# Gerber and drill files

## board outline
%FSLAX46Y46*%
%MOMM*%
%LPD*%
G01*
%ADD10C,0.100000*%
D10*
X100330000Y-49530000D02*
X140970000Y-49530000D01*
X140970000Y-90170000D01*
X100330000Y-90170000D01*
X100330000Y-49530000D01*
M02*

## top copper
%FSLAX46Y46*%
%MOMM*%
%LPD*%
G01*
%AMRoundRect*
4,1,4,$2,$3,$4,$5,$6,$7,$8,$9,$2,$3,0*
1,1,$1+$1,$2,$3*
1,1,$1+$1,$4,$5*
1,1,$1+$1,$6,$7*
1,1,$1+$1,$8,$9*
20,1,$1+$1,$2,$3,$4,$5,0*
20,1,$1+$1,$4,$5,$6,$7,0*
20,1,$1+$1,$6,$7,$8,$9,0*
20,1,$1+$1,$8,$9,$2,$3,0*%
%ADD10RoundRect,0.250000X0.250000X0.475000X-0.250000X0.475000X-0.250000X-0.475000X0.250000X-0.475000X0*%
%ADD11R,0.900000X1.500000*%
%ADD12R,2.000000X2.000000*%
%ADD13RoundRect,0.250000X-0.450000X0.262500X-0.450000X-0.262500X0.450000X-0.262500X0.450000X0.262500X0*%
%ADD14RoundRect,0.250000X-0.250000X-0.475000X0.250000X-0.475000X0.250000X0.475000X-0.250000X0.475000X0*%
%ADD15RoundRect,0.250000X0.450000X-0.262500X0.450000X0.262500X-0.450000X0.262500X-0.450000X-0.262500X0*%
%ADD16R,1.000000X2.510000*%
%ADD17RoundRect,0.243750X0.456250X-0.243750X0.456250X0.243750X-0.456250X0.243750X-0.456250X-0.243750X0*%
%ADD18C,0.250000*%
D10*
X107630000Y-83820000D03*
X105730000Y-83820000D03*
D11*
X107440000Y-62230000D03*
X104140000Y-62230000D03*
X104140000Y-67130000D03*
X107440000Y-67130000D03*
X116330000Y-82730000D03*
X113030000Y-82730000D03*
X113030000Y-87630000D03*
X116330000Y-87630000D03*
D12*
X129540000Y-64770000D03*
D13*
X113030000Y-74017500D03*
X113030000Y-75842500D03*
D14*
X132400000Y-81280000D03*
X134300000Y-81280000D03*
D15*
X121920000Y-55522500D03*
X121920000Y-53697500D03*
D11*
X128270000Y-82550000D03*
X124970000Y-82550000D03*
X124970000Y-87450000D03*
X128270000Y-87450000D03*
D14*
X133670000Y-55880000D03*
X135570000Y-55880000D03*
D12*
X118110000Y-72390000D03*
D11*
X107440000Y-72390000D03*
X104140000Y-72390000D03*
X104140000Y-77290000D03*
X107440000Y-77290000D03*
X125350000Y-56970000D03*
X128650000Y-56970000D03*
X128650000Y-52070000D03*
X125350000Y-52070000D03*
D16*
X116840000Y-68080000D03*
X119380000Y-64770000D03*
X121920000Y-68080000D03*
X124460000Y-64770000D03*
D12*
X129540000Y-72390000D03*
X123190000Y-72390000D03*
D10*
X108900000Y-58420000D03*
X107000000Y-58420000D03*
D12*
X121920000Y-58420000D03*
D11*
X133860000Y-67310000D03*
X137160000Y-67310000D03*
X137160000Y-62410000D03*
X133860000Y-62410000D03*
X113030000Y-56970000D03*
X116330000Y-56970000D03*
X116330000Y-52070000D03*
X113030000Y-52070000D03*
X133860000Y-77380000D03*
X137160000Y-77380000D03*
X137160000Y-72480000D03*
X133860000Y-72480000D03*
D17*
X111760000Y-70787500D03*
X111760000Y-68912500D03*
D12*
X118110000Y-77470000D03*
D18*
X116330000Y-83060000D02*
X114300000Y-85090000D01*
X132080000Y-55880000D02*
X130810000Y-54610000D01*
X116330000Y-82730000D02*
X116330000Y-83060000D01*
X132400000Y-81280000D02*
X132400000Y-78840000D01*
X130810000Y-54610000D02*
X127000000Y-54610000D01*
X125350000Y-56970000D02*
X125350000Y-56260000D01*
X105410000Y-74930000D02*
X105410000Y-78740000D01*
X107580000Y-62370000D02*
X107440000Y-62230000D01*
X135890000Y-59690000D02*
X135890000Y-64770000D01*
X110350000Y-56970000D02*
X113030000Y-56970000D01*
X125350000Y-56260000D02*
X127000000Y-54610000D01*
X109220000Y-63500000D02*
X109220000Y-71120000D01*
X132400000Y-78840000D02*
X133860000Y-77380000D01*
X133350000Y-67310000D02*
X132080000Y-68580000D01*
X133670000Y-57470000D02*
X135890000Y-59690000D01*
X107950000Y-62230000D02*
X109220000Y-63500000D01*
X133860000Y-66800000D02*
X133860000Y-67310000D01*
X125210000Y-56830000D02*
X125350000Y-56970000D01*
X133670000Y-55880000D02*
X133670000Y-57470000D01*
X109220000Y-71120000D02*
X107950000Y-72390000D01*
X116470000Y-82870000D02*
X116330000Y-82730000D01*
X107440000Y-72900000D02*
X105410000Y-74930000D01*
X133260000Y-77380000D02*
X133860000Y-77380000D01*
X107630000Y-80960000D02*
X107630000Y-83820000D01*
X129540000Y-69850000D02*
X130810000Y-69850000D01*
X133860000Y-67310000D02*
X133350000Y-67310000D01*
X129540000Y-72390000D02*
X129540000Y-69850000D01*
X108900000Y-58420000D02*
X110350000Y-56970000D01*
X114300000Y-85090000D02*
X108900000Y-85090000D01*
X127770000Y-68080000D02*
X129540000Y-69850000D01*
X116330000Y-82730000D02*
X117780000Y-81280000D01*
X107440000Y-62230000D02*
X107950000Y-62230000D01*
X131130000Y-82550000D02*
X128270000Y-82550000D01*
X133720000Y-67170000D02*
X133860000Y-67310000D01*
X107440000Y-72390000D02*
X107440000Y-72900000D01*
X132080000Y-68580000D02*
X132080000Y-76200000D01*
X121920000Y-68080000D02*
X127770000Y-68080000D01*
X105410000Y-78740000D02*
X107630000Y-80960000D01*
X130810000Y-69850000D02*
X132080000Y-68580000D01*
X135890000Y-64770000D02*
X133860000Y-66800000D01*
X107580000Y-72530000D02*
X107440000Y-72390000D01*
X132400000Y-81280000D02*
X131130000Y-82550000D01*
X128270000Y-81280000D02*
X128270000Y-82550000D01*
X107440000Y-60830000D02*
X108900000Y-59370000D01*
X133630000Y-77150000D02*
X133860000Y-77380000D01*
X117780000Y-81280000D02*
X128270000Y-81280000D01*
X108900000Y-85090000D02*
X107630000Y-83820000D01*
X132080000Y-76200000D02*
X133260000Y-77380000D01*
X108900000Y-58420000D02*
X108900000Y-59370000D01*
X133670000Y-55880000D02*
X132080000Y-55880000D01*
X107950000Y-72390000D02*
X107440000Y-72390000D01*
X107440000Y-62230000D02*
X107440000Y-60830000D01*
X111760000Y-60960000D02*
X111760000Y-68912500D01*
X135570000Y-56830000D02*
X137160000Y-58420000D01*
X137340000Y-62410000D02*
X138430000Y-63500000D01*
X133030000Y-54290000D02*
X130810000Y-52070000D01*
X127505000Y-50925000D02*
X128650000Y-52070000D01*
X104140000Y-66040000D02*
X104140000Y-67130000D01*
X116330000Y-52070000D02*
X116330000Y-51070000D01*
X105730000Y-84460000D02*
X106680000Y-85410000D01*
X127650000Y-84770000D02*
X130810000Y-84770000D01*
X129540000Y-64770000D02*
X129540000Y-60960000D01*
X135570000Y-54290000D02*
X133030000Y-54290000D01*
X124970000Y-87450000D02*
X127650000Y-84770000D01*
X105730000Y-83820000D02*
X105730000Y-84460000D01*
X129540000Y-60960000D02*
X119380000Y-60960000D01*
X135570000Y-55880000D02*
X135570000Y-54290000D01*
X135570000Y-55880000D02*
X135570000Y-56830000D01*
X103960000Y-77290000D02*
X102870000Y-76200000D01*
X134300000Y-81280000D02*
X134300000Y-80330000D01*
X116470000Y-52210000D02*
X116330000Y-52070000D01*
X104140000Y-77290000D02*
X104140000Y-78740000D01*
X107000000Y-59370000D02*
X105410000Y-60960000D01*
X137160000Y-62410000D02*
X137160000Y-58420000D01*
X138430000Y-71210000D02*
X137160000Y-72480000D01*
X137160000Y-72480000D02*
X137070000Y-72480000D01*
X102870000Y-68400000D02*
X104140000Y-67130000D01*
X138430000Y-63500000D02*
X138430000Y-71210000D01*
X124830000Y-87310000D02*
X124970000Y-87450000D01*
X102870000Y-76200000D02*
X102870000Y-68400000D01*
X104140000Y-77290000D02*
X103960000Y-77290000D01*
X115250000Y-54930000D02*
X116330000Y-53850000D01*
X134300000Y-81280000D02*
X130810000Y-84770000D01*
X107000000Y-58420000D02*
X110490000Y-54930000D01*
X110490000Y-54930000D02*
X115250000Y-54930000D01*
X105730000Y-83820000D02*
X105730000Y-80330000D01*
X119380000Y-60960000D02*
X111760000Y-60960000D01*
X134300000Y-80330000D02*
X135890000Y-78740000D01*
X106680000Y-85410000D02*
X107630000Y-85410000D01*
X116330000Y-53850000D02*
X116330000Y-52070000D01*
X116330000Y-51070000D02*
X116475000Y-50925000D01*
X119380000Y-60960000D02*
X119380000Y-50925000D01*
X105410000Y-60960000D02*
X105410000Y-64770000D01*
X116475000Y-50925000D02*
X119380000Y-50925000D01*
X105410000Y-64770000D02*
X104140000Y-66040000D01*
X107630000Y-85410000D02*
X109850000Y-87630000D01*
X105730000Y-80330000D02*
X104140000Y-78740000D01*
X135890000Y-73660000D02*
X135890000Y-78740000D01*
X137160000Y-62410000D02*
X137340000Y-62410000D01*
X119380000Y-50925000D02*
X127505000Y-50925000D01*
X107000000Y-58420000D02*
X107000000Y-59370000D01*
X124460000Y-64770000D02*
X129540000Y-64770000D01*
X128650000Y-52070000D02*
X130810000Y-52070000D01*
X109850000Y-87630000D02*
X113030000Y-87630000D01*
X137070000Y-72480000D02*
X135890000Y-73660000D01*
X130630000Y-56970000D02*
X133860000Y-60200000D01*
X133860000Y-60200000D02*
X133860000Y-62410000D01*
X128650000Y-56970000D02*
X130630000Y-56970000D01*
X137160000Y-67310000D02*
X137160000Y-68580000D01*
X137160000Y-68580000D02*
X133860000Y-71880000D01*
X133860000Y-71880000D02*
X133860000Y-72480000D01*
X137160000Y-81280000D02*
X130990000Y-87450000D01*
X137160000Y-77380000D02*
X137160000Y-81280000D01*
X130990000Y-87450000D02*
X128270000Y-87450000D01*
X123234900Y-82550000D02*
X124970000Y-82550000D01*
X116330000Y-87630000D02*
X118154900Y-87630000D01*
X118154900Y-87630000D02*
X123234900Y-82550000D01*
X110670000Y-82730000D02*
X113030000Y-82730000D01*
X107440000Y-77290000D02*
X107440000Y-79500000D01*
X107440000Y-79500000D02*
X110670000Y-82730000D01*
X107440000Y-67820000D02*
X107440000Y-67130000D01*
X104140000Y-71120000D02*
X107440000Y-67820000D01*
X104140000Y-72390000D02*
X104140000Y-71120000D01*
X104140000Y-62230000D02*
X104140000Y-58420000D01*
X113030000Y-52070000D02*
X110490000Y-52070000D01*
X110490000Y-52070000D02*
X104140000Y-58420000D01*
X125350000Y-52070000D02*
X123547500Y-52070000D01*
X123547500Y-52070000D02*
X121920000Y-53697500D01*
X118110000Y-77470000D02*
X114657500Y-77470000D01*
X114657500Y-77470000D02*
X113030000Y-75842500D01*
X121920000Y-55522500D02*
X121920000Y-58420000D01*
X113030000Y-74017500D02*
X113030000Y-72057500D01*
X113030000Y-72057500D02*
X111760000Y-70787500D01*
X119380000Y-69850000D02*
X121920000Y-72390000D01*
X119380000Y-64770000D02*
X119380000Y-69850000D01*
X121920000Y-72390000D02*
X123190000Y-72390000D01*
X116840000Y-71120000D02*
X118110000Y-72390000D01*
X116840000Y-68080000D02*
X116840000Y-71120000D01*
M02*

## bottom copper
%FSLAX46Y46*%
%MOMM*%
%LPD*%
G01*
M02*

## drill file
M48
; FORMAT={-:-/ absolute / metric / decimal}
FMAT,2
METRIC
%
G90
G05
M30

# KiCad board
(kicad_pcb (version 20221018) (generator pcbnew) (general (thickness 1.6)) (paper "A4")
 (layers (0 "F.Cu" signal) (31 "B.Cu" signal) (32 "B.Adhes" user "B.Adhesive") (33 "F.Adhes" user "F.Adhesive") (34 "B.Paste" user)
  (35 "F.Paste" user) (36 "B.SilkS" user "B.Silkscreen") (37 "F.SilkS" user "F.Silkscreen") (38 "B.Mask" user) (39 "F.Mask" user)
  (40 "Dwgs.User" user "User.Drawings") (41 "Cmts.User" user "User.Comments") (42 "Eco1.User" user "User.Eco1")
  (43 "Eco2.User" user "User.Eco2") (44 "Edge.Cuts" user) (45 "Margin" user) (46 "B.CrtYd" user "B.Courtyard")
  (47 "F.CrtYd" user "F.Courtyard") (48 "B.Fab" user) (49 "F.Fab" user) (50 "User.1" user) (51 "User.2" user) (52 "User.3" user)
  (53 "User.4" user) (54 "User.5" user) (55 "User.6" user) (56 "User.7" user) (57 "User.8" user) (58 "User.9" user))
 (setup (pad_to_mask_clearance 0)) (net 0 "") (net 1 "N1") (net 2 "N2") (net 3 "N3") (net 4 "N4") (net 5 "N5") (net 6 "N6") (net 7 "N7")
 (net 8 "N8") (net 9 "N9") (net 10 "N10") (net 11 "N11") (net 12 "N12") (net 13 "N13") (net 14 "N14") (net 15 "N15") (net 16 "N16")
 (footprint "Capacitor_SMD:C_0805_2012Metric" (layer "F.Cu") (at 106.68 83.82 180)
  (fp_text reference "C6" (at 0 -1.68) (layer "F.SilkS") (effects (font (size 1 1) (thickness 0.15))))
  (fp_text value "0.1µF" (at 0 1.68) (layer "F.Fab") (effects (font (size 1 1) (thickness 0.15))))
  (pad "1" smd roundrect (at -0.95 0 180) (size 1 1.45) (layers "F.Cu" "F.Paste" "F.Mask") (roundrect_rratio 0.25) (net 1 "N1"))
  (pad "2" smd roundrect (at 0.95 0 180) (size 1 1.45) (layers "F.Cu" "F.Paste" "F.Mask") (roundrect_rratio 0.25) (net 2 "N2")))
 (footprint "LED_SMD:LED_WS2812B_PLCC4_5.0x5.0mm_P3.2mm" (layer "F.Cu") (at 105.79 64.68 -90)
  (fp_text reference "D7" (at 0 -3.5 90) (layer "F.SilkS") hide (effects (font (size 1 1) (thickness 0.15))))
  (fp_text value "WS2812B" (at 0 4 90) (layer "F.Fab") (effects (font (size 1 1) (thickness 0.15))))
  (pad "1" smd rect (at -2.45 -1.65 270) (size 1.5 0.9) (layers "F.Cu" "F.Paste" "F.Mask") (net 1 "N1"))
  (pad "2" smd rect (at -2.45 1.65 270) (size 1.5 0.9) (layers "F.Cu" "F.Paste" "F.Mask") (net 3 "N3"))
  (pad "3" smd rect (at 2.45 1.65 270) (size 1.5 0.9) (layers "F.Cu" "F.Paste" "F.Mask") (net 2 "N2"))
  (pad "4" smd rect (at 2.45 -1.65 270) (size 1.5 0.9) (layers "F.Cu" "F.Paste" "F.Mask") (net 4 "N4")))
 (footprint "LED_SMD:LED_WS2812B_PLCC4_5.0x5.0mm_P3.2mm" (layer "F.Cu") (at 114.68 85.18 -90)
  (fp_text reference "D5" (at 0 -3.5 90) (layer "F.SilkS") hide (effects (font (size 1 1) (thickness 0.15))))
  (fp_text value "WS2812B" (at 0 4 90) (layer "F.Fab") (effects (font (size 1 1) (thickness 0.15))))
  (pad "1" smd rect (at -2.45 -1.65 270) (size 1.5 0.9) (layers "F.Cu" "F.Paste" "F.Mask") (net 1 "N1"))
  (pad "2" smd rect (at -2.45 1.65 270) (size 1.5 0.9) (layers "F.Cu" "F.Paste" "F.Mask") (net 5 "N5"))
  (pad "3" smd rect (at 2.45 1.65 270) (size 1.5 0.9) (layers "F.Cu" "F.Paste" "F.Mask") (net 2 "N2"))
  (pad "4" smd rect (at 2.45 -1.65 270) (size 1.5 0.9) (layers "F.Cu" "F.Paste" "F.Mask") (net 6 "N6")))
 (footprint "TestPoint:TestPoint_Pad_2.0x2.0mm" (layer "F.Cu") (at 129.54 64.77)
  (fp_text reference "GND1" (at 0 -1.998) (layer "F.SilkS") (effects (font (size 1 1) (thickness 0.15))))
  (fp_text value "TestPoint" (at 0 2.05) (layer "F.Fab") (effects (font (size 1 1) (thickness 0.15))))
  (pad "1" smd rect (at 0 0) (size 2 2) (layers "F.Cu" "F.Mask") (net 2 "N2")))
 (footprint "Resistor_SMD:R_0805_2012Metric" (layer "F.Cu") (at 113.03 74.93 -90)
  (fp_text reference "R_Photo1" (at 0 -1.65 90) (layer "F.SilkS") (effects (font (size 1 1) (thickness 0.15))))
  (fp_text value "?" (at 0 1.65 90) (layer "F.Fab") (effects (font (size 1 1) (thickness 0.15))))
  (pad "1" smd roundrect (at -0.9125 0 270) (size 1.025 1.4) (layers "F.Cu" "F.Paste" "F.Mask") (roundrect_rratio 0.243902) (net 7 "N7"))
  (pad "2" smd roundrect (at 0.9125 0 270) (size 1.025 1.4) (layers "F.Cu" "F.Paste" "F.Mask") (roundrect_rratio 0.243902) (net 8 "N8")))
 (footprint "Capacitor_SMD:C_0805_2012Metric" (layer "F.Cu") (at 133.35 81.28)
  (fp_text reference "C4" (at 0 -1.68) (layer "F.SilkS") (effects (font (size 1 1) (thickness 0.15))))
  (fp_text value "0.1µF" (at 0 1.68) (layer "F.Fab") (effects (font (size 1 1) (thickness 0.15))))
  (pad "1" smd roundrect (at -0.95 0) (size 1 1.45) (layers "F.Cu" "F.Paste" "F.Mask") (roundrect_rratio 0.25) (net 1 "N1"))
  (pad "2" smd roundrect (at 0.95 0) (size 1 1.45) (layers "F.Cu" "F.Paste" "F.Mask") (roundrect_rratio 0.25) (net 2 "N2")))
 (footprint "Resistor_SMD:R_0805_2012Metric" (layer "F.Cu") (at 121.92 54.61 90)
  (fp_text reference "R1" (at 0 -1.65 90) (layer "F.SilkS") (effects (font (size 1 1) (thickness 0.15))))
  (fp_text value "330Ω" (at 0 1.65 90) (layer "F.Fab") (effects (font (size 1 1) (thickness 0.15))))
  (pad "1" smd roundrect (at -0.9125 0 90) (size 1.025 1.4) (layers "F.Cu" "F.Paste" "F.Mask") (roundrect_rratio 0.243902) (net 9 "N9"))
  (pad "2" smd roundrect (at 0.9125 0 90) (size 1.025 1.4) (layers "F.Cu" "F.Paste" "F.Mask") (roundrect_rratio 0.243902) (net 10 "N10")))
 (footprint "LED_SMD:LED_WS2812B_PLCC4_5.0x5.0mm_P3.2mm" (layer "F.Cu") (at 126.62 85 -90)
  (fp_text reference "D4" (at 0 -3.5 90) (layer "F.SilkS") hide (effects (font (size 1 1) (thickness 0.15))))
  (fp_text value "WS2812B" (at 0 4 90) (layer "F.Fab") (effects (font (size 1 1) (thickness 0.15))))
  (pad "1" smd rect (at -2.45 -1.65 270) (size 1.5 0.9) (layers "F.Cu" "F.Paste" "F.Mask") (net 1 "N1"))
  (pad "2" smd rect (at -2.45 1.65 270) (size 1.5 0.9) (layers "F.Cu" "F.Paste" "F.Mask") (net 6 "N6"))
  (pad "3" smd rect (at 2.45 1.65 270) (size 1.5 0.9) (layers "F.Cu" "F.Paste" "F.Mask") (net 2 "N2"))
  (pad "4" smd rect (at 2.45 -1.65 270) (size 1.5 0.9) (layers "F.Cu" "F.Paste" "F.Mask") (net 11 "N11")))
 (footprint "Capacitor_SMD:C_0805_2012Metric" (layer "F.Cu") (at 134.62 55.88)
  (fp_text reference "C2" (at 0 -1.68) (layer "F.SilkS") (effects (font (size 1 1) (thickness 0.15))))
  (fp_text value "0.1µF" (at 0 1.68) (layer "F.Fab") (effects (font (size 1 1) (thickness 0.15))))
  (pad "1" smd roundrect (at -0.95 0) (size 1 1.45) (layers "F.Cu" "F.Paste" "F.Mask") (roundrect_rratio 0.25) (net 1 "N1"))
  (pad "2" smd roundrect (at 0.95 0) (size 1 1.45) (layers "F.Cu" "F.Paste" "F.Mask") (roundrect_rratio 0.25) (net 2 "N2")))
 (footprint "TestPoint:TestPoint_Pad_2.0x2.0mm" (layer "F.Cu") (at 118.11 72.39)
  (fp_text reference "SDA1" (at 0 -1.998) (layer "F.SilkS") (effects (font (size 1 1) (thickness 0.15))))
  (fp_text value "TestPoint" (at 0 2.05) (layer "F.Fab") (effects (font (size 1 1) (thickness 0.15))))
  (pad "1" smd rect (at 0 0) (size 2 2) (layers "F.Cu" "F.Mask") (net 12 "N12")))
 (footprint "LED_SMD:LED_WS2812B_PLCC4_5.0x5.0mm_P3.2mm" (layer "F.Cu") (at 105.79 74.84 -90)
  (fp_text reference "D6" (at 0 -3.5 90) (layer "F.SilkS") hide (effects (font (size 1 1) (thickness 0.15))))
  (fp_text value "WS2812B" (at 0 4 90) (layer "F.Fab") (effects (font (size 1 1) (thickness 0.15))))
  (pad "1" smd rect (at -2.45 -1.65 270) (size 1.5 0.9) (layers "F.Cu" "F.Paste" "F.Mask") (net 1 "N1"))
  (pad "2" smd rect (at -2.45 1.65 270) (size 1.5 0.9) (layers "F.Cu" "F.Paste" "F.Mask") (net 4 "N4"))
  (pad "3" smd rect (at 2.45 1.65 270) (size 1.5 0.9) (layers "F.Cu" "F.Paste" "F.Mask") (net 2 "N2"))
  (pad "4" smd rect (at 2.45 -1.65 270) (size 1.5 0.9) (layers "F.Cu" "F.Paste" "F.Mask") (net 5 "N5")))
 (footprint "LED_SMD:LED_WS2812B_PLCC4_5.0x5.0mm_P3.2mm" (layer "F.Cu") (at 127 54.52 90)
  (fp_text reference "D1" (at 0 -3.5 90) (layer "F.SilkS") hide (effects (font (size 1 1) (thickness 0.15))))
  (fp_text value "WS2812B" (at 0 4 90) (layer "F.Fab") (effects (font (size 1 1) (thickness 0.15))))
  (pad "1" smd rect (at -2.45 -1.65 90) (size 1.5 0.9) (layers "F.Cu" "F.Paste" "F.Mask") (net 1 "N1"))
  (pad "2" smd rect (at -2.45 1.65 90) (size 1.5 0.9) (layers "F.Cu" "F.Paste" "F.Mask") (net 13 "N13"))
  (pad "3" smd rect (at 2.45 1.65 90) (size 1.5 0.9) (layers "F.Cu" "F.Paste" "F.Mask") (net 2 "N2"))
  (pad "4" smd rect (at 2.45 -1.65 90) (size 1.5 0.9) (layers "F.Cu" "F.Paste" "F.Mask") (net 10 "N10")))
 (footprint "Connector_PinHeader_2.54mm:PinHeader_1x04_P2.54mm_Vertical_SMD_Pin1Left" (layer "F.Cu") (at 120.65 66.425 90)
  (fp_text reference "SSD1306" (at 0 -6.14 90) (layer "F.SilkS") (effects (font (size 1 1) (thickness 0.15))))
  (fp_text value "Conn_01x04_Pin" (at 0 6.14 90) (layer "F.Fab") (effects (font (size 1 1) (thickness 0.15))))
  (pad "1" smd rect (at -1.655 -3.81 90) (size 2.51 1) (layers "F.Cu" "F.Paste" "F.Mask") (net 12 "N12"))
  (pad "2" smd rect (at 1.655 -1.27 90) (size 2.51 1) (layers "F.Cu" "F.Paste" "F.Mask") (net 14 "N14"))
  (pad "3" smd rect (at -1.655 1.27 90) (size 2.51 1) (layers "F.Cu" "F.Paste" "F.Mask") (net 1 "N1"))
  (pad "4" smd rect (at 1.655 3.81 90) (size 2.51 1) (layers "F.Cu" "F.Paste" "F.Mask") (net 2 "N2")))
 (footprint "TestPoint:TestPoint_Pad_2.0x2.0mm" (layer "F.Cu") (at 129.54 72.39)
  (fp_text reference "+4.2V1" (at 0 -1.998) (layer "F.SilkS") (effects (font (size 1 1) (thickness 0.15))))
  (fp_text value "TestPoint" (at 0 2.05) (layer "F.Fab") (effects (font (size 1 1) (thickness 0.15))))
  (pad "1" smd rect (at 0 0) (size 2 2) (layers "F.Cu" "F.Mask") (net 1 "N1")))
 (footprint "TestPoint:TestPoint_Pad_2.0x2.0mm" (layer "F.Cu") (at 123.19 72.39)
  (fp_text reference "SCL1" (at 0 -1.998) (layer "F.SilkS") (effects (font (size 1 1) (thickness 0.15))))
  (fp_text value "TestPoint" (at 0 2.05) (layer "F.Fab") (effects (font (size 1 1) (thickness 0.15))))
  (pad "1" smd rect (at 0 0) (size 2 2) (layers "F.Cu" "F.Mask") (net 14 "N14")))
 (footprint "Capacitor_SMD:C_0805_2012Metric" (layer "F.Cu") (at 107.95 58.42 180)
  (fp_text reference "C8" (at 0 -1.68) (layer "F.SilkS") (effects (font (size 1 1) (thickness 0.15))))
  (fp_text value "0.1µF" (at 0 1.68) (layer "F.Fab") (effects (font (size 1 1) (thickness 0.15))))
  (pad "1" smd roundrect (at -0.95 0 180) (size 1 1.45) (layers "F.Cu" "F.Paste" "F.Mask") (roundrect_rratio 0.25) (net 1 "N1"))
  (pad "2" smd roundrect (at 0.95 0 180) (size 1 1.45) (layers "F.Cu" "F.Paste" "F.Mask") (roundrect_rratio 0.25) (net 2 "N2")))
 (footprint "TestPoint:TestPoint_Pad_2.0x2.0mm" (layer "F.Cu") (at 121.92 58.42)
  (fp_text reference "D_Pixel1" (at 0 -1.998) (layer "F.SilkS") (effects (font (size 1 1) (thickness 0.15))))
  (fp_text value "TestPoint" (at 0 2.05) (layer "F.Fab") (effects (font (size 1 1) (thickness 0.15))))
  (pad "1" smd rect (at 0 0) (size 2 2) (layers "F.Cu" "F.Mask") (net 9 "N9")))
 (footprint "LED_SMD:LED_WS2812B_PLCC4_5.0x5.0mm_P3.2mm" (layer "F.Cu") (at 135.51 64.86 90)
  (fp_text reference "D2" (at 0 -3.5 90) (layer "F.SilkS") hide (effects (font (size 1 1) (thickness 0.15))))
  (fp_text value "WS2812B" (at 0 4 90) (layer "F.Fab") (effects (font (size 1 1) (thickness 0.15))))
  (pad "1" smd rect (at -2.45 -1.65 90) (size 1.5 0.9) (layers "F.Cu" "F.Paste" "F.Mask") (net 1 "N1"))
  (pad "2" smd rect (at -2.45 1.65 90) (size 1.5 0.9) (layers "F.Cu" "F.Paste" "F.Mask") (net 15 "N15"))
  (pad "3" smd rect (at 2.45 1.65 90) (size 1.5 0.9) (layers "F.Cu" "F.Paste" "F.Mask") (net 2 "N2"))
  (pad "4" smd rect (at 2.45 -1.65 90) (size 1.5 0.9) (layers "F.Cu" "F.Paste" "F.Mask") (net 13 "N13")))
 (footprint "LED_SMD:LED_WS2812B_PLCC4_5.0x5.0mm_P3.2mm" (layer "F.Cu") (at 114.68 54.52 90)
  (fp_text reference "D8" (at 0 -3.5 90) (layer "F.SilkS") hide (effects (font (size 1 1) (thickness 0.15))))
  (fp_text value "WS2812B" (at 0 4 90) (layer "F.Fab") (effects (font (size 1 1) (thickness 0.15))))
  (pad "1" smd rect (at -2.45 -1.65 90) (size 1.5 0.9) (layers "F.Cu" "F.Paste" "F.Mask") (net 1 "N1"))
  (pad "2" smd rect (at -2.45 1.65 90) (size 1.5 0.9) (layers "F.Cu" "F.Paste" "F.Mask") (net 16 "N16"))
  (pad "3" smd rect (at 2.45 1.65 90) (size 1.5 0.9) (layers "F.Cu" "F.Paste" "F.Mask") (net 2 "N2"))
  (pad "4" smd rect (at 2.45 -1.65 90) (size 1.5 0.9) (layers "F.Cu" "F.Paste" "F.Mask") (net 3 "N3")))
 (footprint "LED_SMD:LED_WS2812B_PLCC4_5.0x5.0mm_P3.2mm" (layer "F.Cu") (at 135.51 74.93 90)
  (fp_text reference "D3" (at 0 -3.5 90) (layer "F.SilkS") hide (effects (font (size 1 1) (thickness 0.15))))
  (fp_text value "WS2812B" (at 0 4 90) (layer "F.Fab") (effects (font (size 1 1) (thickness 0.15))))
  (pad "1" smd rect (at -2.45 -1.65 90) (size 1.5 0.9) (layers "F.Cu" "F.Paste" "F.Mask") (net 1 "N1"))
  (pad "2" smd rect (at -2.45 1.65 90) (size 1.5 0.9) (layers "F.Cu" "F.Paste" "F.Mask") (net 11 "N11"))
  (pad "3" smd rect (at 2.45 1.65 90) (size 1.5 0.9) (layers "F.Cu" "F.Paste" "F.Mask") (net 2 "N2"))
  (pad "4" smd rect (at 2.45 -1.65 90) (size 1.5 0.9) (layers "F.Cu" "F.Paste" "F.Mask") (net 15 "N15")))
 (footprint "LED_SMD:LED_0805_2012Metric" (layer "F.Cu") (at 111.76 69.85 90)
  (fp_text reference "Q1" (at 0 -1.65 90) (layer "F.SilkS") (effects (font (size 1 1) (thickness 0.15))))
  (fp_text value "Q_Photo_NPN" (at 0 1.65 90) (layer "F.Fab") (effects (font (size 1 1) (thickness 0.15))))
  (pad "1" smd roundrect (at -0.9375 0 90) (size 0.975 1.4) (layers "F.Cu" "F.Paste" "F.Mask") (roundrect_rratio 0.25) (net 7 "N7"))
  (pad "2" smd roundrect (at 0.9375 0 90) (size 0.975 1.4) (layers "F.Cu" "F.Paste" "F.Mask") (roundrect_rratio 0.25) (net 2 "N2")))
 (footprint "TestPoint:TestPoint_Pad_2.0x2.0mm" (layer "F.Cu") (at 118.11 77.47)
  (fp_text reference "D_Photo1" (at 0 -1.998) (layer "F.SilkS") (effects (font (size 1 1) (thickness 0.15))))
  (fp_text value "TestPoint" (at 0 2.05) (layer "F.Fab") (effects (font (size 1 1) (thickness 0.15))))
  (pad "1" smd rect (at 0 0) (size 2 2) (layers "F.Cu" "F.Mask") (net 8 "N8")))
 (gr_rect (start 100.33 49.53) (end 140.97 90.17) (stroke (width 0.1) (type default)) (fill none) (layer "Edge.Cuts"))
 (segment (start 116.33 83.06) (end 114.3 85.09) (width 0.25) (layer "F.Cu") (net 1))
 (segment (start 132.08 55.88) (end 130.81 54.61) (width 0.25) (layer "F.Cu") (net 1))
 (segment (start 116.33 82.73) (end 116.33 83.06) (width 0.25) (layer "F.Cu") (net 1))
 (segment (start 132.4 81.28) (end 132.4 78.84) (width 0.25) (layer "F.Cu") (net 1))
 (segment (start 130.81 54.61) (end 127 54.61) (width 0.25) (layer "F.Cu") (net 1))
 (segment (start 125.35 56.97) (end 125.35 56.26) (width 0.25) (layer "F.Cu") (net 1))
 (segment (start 105.41 74.93) (end 105.41 78.74) (width 0.25) (layer "F.Cu") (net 1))
 (segment (start 107.58 62.37) (end 107.44 62.23) (width 0.25) (layer "F.Cu") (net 1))
 (segment (start 135.89 59.69) (end 135.89 64.77) (width 0.25) (layer "F.Cu") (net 1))
 (segment (start 110.35 56.97) (end 113.03 56.97) (width 0.25) (layer "F.Cu") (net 1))
 (segment (start 125.35 56.26) (end 127 54.61) (width 0.25) (layer "F.Cu") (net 1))
 (segment (start 109.22 63.5) (end 109.22 71.12) (width 0.25) (layer "F.Cu") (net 1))
 (segment (start 132.4 78.84) (end 133.86 77.38) (width 0.25) (layer "F.Cu") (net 1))
 (segment (start 133.35 67.31) (end 132.08 68.58) (width 0.25) (layer "F.Cu") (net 1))
 (segment (start 133.67 57.47) (end 135.89 59.69) (width 0.25) (layer "F.Cu") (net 1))
 (segment (start 107.95 62.23) (end 109.22 63.5) (width 0.25) (layer "F.Cu") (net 1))
 (segment (start 133.86 66.8) (end 133.86 67.31) (width 0.25) (layer "F.Cu") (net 1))
 (segment (start 125.21 56.83) (end 125.35 56.97) (width 0.25) (layer "F.Cu") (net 1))
 (segment (start 133.67 55.88) (end 133.67 57.47) (width 0.25) (layer "F.Cu") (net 1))
 (segment (start 109.22 71.12) (end 107.95 72.39) (width 0.25) (layer "F.Cu") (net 1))
 (segment (start 116.47 82.87) (end 116.33 82.73) (width 0.25) (layer "F.Cu") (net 1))
 (segment (start 107.44 72.9) (end 105.41 74.93) (width 0.25) (layer "F.Cu") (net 1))
 (segment (start 133.26 77.38) (end 133.86 77.38) (width 0.25) (layer "F.Cu") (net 1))
 (segment (start 107.63 80.96) (end 107.63 83.82) (width 0.25) (layer "F.Cu") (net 1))
 (segment (start 129.54 69.85) (end 130.81 69.85) (width 0.25) (layer "F.Cu") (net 1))
 (segment (start 133.86 67.31) (end 133.35 67.31) (width 0.25) (layer "F.Cu") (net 1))
 (segment (start 129.54 72.39) (end 129.54 69.85) (width 0.25) (layer "F.Cu") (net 1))
 (segment (start 108.9 58.42) (end 110.35 56.97) (width 0.25) (layer "F.Cu") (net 1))
 (segment (start 114.3 85.09) (end 108.9 85.09) (width 0.25) (layer "F.Cu") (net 1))
 (segment (start 127.77 68.08) (end 129.54 69.85) (width 0.25) (layer "F.Cu") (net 1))
 (segment (start 116.33 82.73) (end 117.78 81.28) (width 0.25) (layer "F.Cu") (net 1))
 (segment (start 107.44 62.23) (end 107.95 62.23) (width 0.25) (layer "F.Cu") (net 1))
 (segment (start 131.13 82.55) (end 128.27 82.55) (width 0.25) (layer "F.Cu") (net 1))
 (segment (start 133.72 67.17) (end 133.86 67.31) (width 0.25) (layer "F.Cu") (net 1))
 (segment (start 107.44 72.39) (end 107.44 72.9) (width 0.25) (layer "F.Cu") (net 1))
 (segment (start 132.08 68.58) (end 132.08 76.2) (width 0.25) (layer "F.Cu") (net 1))
 (segment (start 121.92 68.08) (end 127.77 68.08) (width 0.25) (layer "F.Cu") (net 1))
 (segment (start 105.41 78.74) (end 107.63 80.96) (width 0.25) (layer "F.Cu") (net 1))
 (segment (start 130.81 69.85) (end 132.08 68.58) (width 0.25) (layer "F.Cu") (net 1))
 (segment (start 135.89 64.77) (end 133.86 66.8) (width 0.25) (layer "F.Cu") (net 1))
 (segment (start 107.58 72.53) (end 107.44 72.39) (width 0.25) (layer "F.Cu") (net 1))
 (segment (start 132.4 81.28) (end 131.13 82.55) (width 0.25) (layer "F.Cu") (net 1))
 (segment (start 128.27 81.28) (end 128.27 82.55) (width 0.25) (layer "F.Cu") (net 1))
 (segment (start 107.44 60.83) (end 108.9 59.37) (width 0.25) (layer "F.Cu") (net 1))
 (segment (start 133.63 77.15) (end 133.86 77.38) (width 0.25) (layer "F.Cu") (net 1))
 (segment (start 117.78 81.28) (end 128.27 81.28) (width 0.25) (layer "F.Cu") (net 1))
 (segment (start 108.9 85.09) (end 107.63 83.82) (width 0.25) (layer "F.Cu") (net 1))
 (segment (start 132.08 76.2) (end 133.26 77.38) (width 0.25) (layer "F.Cu") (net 1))
 (segment (start 108.9 58.42) (end 108.9 59.37) (width 0.25) (layer "F.Cu") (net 1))
 (segment (start 133.67 55.88) (end 132.08 55.88) (width 0.25) (layer "F.Cu") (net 1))
 (segment (start 107.95 72.39) (end 107.44 72.39) (width 0.25) (layer "F.Cu") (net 1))
 (segment (start 107.44 62.23) (end 107.44 60.83) (width 0.25) (layer "F.Cu") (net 1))
 (segment (start 111.76 60.96) (end 111.76 68.9125) (width 0.25) (layer "F.Cu") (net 2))
 (segment (start 135.57 56.83) (end 137.16 58.42) (width 0.25) (layer "F.Cu") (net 2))
 (segment (start 137.34 62.41) (end 138.43 63.5) (width 0.25) (layer "F.Cu") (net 2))
 (segment (start 133.03 54.29) (end 130.81 52.07) (width 0.25) (layer "F.Cu") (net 2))
 (segment (start 127.505 50.925) (end 128.65 52.07) (width 0.25) (layer "F.Cu") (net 2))
 (segment (start 104.14 66.04) (end 104.14 67.13) (width 0.25) (layer "F.Cu") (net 2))
 (segment (start 116.33 52.07) (end 116.33 51.07) (width 0.25) (layer "F.Cu") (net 2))
 (segment (start 105.73 84.46) (end 106.68 85.41) (width 0.25) (layer "F.Cu") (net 2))
 (segment (start 127.65 84.77) (end 130.81 84.77) (width 0.25) (layer "F.Cu") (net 2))
 (segment (start 129.54 64.77) (end 129.54 60.96) (width 0.25) (layer "F.Cu") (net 2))
 (segment (start 135.57 54.29) (end 133.03 54.29) (width 0.25) (layer "F.Cu") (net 2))
 (segment (start 124.97 87.45) (end 127.65 84.77) (width 0.25) (layer "F.Cu") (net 2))
 (segment (start 105.73 83.82) (end 105.73 84.46) (width 0.25) (layer "F.Cu") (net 2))
 (segment (start 129.54 60.96) (end 119.38 60.96) (width 0.25) (layer "F.Cu") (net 2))
 (segment (start 135.57 55.88) (end 135.57 54.29) (width 0.25) (layer "F.Cu") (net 2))
 (segment (start 135.57 55.88) (end 135.57 56.83) (width 0.25) (layer "F.Cu") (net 2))
 (segment (start 103.96 77.29) (end 102.87 76.2) (width 0.25) (layer "F.Cu") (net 2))
 (segment (start 134.3 81.28) (end 134.3 80.33) (width 0.25) (layer "F.Cu") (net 2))
 (segment (start 116.47 52.21) (end 116.33 52.07) (width 0.25) (layer "F.Cu") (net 2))
 (segment (start 104.14 77.29) (end 104.14 78.74) (width 0.25) (layer "F.Cu") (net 2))
 (segment (start 107 59.37) (end 105.41 60.96) (width 0.25) (layer "F.Cu") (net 2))
 (segment (start 137.16 62.41) (end 137.16 58.42) (width 0.25) (layer "F.Cu") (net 2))
 (segment (start 138.43 71.21) (end 137.16 72.48) (width 0.25) (layer "F.Cu") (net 2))
 (segment (start 137.16 72.48) (end 137.07 72.48) (width 0.25) (layer "F.Cu") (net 2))
 (segment (start 102.87 68.4) (end 104.14 67.13) (width 0.25) (layer "F.Cu") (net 2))
 (segment (start 138.43 63.5) (end 138.43 71.21) (width 0.25) (layer "F.Cu") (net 2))
 (segment (start 124.83 87.31) (end 124.97 87.45) (width 0.25) (layer "F.Cu") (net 2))
 (segment (start 102.87 76.2) (end 102.87 68.4) (width 0.25) (layer "F.Cu") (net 2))
 (segment (start 104.14 77.29) (end 103.96 77.29) (width 0.25) (layer "F.Cu") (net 2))
 (segment (start 115.25 54.93) (end 116.33 53.85) (width 0.25) (layer "F.Cu") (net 2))
 (segment (start 134.3 81.28) (end 130.81 84.77) (width 0.25) (layer "F.Cu") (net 2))
 (segment (start 107 58.42) (end 110.49 54.93) (width 0.25) (layer "F.Cu") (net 2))
 (segment (start 110.49 54.93) (end 115.25 54.93) (width 0.25) (layer "F.Cu") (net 2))
 (segment (start 105.73 83.82) (end 105.73 80.33) (width 0.25) (layer "F.Cu") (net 2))
 (segment (start 119.38 60.96) (end 111.76 60.96) (width 0.25) (layer "F.Cu") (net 2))
 (segment (start 134.3 80.33) (end 135.89 78.74) (width 0.25) (layer "F.Cu") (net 2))
 (segment (start 106.68 85.41) (end 107.63 85.41) (width 0.25) (layer "F.Cu") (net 2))
 (segment (start 116.33 53.85) (end 116.33 52.07) (width 0.25) (layer "F.Cu") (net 2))
 (segment (start 116.33 51.07) (end 116.475 50.925) (width 0.25) (layer "F.Cu") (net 2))
 (segment (start 119.38 60.96) (end 119.38 50.925) (width 0.25) (layer "F.Cu") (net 2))
 (segment (start 105.41 60.96) (end 105.41 64.77) (width 0.25) (layer "F.Cu") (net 2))
 (segment (start 116.475 50.925) (end 119.38 50.925) (width 0.25) (layer "F.Cu") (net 2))
 (segment (start 105.41 64.77) (end 104.14 66.04) (width 0.25) (layer "F.Cu") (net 2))
 (segment (start 107.63 85.41) (end 109.85 87.63) (width 0.25) (layer "F.Cu") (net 2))
 (segment (start 105.73 80.33) (end 104.14 78.74) (width 0.25) (layer "F.Cu") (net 2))
 (segment (start 135.89 73.66) (end 135.89 78.74) (width 0.25) (layer "F.Cu") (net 2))
 (segment (start 137.16 62.41) (end 137.34 62.41) (width 0.25) (layer "F.Cu") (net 2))
 (segment (start 119.38 50.925) (end 127.505 50.925) (width 0.25) (layer "F.Cu") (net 2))
 (segment (start 107 58.42) (end 107 59.37) (width 0.25) (layer "F.Cu") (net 2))
 (segment (start 124.46 64.77) (end 129.54 64.77) (width 0.25) (layer "F.Cu") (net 2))
 (segment (start 128.65 52.07) (end 130.81 52.07) (width 0.25) (layer "F.Cu") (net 2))
 (segment (start 109.85 87.63) (end 113.03 87.63) (width 0.25) (layer "F.Cu") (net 2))
 (segment (start 137.07 72.48) (end 135.89 73.66) (width 0.25) (layer "F.Cu") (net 2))
 (segment (start 130.63 56.97) (end 133.86 60.2) (width 0.25) (layer "F.Cu") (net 13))
 (segment (start 133.86 60.2) (end 133.86 62.41) (width 0.25) (layer "F.Cu") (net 13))
 (segment (start 128.65 56.97) (end 130.63 56.97) (width 0.25) (layer "F.Cu") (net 13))
 (segment (start 137.16 67.31) (end 137.16 68.58) (width 0.25) (layer "F.Cu") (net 15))
 (segment (start 137.16 68.58) (end 133.86 71.88) (width 0.25) (layer "F.Cu") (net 15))
 (segment (start 133.86 71.88) (end 133.86 72.48) (width 0.25) (layer "F.Cu") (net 15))
 (segment (start 137.16 81.28) (end 130.99 87.45) (width 0.25) (layer "F.Cu") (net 11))
 (segment (start 137.16 77.38) (end 137.16 81.28) (width 0.25) (layer "F.Cu") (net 11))
 (segment (start 130.99 87.45) (end 128.27 87.45) (width 0.25) (layer "F.Cu") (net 11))
 (segment (start 123.2349 82.55) (end 124.97 82.55) (width 0.25) (layer "F.Cu") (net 6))
 (segment (start 116.33 87.63) (end 118.1549 87.63) (width 0.25) (layer "F.Cu") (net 6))
 (segment (start 118.1549 87.63) (end 123.2349 82.55) (width 0.25) (layer "F.Cu") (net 6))
 (segment (start 110.67 82.73) (end 113.03 82.73) (width 0.25) (layer "F.Cu") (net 5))
 (segment (start 107.44 77.29) (end 107.44 79.5) (width 0.25) (layer "F.Cu") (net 5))
 (segment (start 107.44 79.5) (end 110.67 82.73) (width 0.25) (layer "F.Cu") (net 5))
 (segment (start 107.44 67.82) (end 107.44 67.13) (width 0.25) (layer "F.Cu") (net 4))
 (segment (start 104.14 71.12) (end 107.44 67.82) (width 0.25) (layer "F.Cu") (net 4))
 (segment (start 104.14 72.39) (end 104.14 71.12) (width 0.25) (layer "F.Cu") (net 4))
 (segment (start 104.14 62.23) (end 104.14 58.42) (width 0.25) (layer "F.Cu") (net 3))
 (segment (start 113.03 52.07) (end 110.49 52.07) (width 0.25) (layer "F.Cu") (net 3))
 (segment (start 110.49 52.07) (end 104.14 58.42) (width 0.25) (layer "F.Cu") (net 3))
 (segment (start 125.35 52.07) (end 123.5475 52.07) (width 0.25) (layer "F.Cu") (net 10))
 (segment (start 123.5475 52.07) (end 121.92 53.6975) (width 0.25) (layer "F.Cu") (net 10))
 (segment (start 118.11 77.47) (end 114.6575 77.47) (width 0.25) (layer "F.Cu") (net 8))
 (segment (start 114.6575 77.47) (end 113.03 75.8425) (width 0.25) (layer "F.Cu") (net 8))
 (segment (start 121.92 55.5225) (end 121.92 58.42) (width 0.25) (layer "F.Cu") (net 9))
 (segment (start 113.03 74.0175) (end 113.03 72.0575) (width 0.25) (layer "F.Cu") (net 7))
 (segment (start 113.03 72.0575) (end 111.76 70.7875) (width 0.25) (layer "F.Cu") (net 7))
 (segment (start 119.38 69.85) (end 121.92 72.39) (width 0.25) (layer "F.Cu") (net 14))
 (segment (start 119.38 64.77) (end 119.38 69.85) (width 0.25) (layer "F.Cu") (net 14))
 (segment (start 121.92 72.39) (end 123.19 72.39) (width 0.25) (layer "F.Cu") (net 14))
 (segment (start 116.84 71.12) (end 118.11 72.39) (width 0.25) (layer "F.Cu") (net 12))
 (segment (start 116.84 68.08) (end 116.84 71.12) (width 0.25) (layer "F.Cu") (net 12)))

